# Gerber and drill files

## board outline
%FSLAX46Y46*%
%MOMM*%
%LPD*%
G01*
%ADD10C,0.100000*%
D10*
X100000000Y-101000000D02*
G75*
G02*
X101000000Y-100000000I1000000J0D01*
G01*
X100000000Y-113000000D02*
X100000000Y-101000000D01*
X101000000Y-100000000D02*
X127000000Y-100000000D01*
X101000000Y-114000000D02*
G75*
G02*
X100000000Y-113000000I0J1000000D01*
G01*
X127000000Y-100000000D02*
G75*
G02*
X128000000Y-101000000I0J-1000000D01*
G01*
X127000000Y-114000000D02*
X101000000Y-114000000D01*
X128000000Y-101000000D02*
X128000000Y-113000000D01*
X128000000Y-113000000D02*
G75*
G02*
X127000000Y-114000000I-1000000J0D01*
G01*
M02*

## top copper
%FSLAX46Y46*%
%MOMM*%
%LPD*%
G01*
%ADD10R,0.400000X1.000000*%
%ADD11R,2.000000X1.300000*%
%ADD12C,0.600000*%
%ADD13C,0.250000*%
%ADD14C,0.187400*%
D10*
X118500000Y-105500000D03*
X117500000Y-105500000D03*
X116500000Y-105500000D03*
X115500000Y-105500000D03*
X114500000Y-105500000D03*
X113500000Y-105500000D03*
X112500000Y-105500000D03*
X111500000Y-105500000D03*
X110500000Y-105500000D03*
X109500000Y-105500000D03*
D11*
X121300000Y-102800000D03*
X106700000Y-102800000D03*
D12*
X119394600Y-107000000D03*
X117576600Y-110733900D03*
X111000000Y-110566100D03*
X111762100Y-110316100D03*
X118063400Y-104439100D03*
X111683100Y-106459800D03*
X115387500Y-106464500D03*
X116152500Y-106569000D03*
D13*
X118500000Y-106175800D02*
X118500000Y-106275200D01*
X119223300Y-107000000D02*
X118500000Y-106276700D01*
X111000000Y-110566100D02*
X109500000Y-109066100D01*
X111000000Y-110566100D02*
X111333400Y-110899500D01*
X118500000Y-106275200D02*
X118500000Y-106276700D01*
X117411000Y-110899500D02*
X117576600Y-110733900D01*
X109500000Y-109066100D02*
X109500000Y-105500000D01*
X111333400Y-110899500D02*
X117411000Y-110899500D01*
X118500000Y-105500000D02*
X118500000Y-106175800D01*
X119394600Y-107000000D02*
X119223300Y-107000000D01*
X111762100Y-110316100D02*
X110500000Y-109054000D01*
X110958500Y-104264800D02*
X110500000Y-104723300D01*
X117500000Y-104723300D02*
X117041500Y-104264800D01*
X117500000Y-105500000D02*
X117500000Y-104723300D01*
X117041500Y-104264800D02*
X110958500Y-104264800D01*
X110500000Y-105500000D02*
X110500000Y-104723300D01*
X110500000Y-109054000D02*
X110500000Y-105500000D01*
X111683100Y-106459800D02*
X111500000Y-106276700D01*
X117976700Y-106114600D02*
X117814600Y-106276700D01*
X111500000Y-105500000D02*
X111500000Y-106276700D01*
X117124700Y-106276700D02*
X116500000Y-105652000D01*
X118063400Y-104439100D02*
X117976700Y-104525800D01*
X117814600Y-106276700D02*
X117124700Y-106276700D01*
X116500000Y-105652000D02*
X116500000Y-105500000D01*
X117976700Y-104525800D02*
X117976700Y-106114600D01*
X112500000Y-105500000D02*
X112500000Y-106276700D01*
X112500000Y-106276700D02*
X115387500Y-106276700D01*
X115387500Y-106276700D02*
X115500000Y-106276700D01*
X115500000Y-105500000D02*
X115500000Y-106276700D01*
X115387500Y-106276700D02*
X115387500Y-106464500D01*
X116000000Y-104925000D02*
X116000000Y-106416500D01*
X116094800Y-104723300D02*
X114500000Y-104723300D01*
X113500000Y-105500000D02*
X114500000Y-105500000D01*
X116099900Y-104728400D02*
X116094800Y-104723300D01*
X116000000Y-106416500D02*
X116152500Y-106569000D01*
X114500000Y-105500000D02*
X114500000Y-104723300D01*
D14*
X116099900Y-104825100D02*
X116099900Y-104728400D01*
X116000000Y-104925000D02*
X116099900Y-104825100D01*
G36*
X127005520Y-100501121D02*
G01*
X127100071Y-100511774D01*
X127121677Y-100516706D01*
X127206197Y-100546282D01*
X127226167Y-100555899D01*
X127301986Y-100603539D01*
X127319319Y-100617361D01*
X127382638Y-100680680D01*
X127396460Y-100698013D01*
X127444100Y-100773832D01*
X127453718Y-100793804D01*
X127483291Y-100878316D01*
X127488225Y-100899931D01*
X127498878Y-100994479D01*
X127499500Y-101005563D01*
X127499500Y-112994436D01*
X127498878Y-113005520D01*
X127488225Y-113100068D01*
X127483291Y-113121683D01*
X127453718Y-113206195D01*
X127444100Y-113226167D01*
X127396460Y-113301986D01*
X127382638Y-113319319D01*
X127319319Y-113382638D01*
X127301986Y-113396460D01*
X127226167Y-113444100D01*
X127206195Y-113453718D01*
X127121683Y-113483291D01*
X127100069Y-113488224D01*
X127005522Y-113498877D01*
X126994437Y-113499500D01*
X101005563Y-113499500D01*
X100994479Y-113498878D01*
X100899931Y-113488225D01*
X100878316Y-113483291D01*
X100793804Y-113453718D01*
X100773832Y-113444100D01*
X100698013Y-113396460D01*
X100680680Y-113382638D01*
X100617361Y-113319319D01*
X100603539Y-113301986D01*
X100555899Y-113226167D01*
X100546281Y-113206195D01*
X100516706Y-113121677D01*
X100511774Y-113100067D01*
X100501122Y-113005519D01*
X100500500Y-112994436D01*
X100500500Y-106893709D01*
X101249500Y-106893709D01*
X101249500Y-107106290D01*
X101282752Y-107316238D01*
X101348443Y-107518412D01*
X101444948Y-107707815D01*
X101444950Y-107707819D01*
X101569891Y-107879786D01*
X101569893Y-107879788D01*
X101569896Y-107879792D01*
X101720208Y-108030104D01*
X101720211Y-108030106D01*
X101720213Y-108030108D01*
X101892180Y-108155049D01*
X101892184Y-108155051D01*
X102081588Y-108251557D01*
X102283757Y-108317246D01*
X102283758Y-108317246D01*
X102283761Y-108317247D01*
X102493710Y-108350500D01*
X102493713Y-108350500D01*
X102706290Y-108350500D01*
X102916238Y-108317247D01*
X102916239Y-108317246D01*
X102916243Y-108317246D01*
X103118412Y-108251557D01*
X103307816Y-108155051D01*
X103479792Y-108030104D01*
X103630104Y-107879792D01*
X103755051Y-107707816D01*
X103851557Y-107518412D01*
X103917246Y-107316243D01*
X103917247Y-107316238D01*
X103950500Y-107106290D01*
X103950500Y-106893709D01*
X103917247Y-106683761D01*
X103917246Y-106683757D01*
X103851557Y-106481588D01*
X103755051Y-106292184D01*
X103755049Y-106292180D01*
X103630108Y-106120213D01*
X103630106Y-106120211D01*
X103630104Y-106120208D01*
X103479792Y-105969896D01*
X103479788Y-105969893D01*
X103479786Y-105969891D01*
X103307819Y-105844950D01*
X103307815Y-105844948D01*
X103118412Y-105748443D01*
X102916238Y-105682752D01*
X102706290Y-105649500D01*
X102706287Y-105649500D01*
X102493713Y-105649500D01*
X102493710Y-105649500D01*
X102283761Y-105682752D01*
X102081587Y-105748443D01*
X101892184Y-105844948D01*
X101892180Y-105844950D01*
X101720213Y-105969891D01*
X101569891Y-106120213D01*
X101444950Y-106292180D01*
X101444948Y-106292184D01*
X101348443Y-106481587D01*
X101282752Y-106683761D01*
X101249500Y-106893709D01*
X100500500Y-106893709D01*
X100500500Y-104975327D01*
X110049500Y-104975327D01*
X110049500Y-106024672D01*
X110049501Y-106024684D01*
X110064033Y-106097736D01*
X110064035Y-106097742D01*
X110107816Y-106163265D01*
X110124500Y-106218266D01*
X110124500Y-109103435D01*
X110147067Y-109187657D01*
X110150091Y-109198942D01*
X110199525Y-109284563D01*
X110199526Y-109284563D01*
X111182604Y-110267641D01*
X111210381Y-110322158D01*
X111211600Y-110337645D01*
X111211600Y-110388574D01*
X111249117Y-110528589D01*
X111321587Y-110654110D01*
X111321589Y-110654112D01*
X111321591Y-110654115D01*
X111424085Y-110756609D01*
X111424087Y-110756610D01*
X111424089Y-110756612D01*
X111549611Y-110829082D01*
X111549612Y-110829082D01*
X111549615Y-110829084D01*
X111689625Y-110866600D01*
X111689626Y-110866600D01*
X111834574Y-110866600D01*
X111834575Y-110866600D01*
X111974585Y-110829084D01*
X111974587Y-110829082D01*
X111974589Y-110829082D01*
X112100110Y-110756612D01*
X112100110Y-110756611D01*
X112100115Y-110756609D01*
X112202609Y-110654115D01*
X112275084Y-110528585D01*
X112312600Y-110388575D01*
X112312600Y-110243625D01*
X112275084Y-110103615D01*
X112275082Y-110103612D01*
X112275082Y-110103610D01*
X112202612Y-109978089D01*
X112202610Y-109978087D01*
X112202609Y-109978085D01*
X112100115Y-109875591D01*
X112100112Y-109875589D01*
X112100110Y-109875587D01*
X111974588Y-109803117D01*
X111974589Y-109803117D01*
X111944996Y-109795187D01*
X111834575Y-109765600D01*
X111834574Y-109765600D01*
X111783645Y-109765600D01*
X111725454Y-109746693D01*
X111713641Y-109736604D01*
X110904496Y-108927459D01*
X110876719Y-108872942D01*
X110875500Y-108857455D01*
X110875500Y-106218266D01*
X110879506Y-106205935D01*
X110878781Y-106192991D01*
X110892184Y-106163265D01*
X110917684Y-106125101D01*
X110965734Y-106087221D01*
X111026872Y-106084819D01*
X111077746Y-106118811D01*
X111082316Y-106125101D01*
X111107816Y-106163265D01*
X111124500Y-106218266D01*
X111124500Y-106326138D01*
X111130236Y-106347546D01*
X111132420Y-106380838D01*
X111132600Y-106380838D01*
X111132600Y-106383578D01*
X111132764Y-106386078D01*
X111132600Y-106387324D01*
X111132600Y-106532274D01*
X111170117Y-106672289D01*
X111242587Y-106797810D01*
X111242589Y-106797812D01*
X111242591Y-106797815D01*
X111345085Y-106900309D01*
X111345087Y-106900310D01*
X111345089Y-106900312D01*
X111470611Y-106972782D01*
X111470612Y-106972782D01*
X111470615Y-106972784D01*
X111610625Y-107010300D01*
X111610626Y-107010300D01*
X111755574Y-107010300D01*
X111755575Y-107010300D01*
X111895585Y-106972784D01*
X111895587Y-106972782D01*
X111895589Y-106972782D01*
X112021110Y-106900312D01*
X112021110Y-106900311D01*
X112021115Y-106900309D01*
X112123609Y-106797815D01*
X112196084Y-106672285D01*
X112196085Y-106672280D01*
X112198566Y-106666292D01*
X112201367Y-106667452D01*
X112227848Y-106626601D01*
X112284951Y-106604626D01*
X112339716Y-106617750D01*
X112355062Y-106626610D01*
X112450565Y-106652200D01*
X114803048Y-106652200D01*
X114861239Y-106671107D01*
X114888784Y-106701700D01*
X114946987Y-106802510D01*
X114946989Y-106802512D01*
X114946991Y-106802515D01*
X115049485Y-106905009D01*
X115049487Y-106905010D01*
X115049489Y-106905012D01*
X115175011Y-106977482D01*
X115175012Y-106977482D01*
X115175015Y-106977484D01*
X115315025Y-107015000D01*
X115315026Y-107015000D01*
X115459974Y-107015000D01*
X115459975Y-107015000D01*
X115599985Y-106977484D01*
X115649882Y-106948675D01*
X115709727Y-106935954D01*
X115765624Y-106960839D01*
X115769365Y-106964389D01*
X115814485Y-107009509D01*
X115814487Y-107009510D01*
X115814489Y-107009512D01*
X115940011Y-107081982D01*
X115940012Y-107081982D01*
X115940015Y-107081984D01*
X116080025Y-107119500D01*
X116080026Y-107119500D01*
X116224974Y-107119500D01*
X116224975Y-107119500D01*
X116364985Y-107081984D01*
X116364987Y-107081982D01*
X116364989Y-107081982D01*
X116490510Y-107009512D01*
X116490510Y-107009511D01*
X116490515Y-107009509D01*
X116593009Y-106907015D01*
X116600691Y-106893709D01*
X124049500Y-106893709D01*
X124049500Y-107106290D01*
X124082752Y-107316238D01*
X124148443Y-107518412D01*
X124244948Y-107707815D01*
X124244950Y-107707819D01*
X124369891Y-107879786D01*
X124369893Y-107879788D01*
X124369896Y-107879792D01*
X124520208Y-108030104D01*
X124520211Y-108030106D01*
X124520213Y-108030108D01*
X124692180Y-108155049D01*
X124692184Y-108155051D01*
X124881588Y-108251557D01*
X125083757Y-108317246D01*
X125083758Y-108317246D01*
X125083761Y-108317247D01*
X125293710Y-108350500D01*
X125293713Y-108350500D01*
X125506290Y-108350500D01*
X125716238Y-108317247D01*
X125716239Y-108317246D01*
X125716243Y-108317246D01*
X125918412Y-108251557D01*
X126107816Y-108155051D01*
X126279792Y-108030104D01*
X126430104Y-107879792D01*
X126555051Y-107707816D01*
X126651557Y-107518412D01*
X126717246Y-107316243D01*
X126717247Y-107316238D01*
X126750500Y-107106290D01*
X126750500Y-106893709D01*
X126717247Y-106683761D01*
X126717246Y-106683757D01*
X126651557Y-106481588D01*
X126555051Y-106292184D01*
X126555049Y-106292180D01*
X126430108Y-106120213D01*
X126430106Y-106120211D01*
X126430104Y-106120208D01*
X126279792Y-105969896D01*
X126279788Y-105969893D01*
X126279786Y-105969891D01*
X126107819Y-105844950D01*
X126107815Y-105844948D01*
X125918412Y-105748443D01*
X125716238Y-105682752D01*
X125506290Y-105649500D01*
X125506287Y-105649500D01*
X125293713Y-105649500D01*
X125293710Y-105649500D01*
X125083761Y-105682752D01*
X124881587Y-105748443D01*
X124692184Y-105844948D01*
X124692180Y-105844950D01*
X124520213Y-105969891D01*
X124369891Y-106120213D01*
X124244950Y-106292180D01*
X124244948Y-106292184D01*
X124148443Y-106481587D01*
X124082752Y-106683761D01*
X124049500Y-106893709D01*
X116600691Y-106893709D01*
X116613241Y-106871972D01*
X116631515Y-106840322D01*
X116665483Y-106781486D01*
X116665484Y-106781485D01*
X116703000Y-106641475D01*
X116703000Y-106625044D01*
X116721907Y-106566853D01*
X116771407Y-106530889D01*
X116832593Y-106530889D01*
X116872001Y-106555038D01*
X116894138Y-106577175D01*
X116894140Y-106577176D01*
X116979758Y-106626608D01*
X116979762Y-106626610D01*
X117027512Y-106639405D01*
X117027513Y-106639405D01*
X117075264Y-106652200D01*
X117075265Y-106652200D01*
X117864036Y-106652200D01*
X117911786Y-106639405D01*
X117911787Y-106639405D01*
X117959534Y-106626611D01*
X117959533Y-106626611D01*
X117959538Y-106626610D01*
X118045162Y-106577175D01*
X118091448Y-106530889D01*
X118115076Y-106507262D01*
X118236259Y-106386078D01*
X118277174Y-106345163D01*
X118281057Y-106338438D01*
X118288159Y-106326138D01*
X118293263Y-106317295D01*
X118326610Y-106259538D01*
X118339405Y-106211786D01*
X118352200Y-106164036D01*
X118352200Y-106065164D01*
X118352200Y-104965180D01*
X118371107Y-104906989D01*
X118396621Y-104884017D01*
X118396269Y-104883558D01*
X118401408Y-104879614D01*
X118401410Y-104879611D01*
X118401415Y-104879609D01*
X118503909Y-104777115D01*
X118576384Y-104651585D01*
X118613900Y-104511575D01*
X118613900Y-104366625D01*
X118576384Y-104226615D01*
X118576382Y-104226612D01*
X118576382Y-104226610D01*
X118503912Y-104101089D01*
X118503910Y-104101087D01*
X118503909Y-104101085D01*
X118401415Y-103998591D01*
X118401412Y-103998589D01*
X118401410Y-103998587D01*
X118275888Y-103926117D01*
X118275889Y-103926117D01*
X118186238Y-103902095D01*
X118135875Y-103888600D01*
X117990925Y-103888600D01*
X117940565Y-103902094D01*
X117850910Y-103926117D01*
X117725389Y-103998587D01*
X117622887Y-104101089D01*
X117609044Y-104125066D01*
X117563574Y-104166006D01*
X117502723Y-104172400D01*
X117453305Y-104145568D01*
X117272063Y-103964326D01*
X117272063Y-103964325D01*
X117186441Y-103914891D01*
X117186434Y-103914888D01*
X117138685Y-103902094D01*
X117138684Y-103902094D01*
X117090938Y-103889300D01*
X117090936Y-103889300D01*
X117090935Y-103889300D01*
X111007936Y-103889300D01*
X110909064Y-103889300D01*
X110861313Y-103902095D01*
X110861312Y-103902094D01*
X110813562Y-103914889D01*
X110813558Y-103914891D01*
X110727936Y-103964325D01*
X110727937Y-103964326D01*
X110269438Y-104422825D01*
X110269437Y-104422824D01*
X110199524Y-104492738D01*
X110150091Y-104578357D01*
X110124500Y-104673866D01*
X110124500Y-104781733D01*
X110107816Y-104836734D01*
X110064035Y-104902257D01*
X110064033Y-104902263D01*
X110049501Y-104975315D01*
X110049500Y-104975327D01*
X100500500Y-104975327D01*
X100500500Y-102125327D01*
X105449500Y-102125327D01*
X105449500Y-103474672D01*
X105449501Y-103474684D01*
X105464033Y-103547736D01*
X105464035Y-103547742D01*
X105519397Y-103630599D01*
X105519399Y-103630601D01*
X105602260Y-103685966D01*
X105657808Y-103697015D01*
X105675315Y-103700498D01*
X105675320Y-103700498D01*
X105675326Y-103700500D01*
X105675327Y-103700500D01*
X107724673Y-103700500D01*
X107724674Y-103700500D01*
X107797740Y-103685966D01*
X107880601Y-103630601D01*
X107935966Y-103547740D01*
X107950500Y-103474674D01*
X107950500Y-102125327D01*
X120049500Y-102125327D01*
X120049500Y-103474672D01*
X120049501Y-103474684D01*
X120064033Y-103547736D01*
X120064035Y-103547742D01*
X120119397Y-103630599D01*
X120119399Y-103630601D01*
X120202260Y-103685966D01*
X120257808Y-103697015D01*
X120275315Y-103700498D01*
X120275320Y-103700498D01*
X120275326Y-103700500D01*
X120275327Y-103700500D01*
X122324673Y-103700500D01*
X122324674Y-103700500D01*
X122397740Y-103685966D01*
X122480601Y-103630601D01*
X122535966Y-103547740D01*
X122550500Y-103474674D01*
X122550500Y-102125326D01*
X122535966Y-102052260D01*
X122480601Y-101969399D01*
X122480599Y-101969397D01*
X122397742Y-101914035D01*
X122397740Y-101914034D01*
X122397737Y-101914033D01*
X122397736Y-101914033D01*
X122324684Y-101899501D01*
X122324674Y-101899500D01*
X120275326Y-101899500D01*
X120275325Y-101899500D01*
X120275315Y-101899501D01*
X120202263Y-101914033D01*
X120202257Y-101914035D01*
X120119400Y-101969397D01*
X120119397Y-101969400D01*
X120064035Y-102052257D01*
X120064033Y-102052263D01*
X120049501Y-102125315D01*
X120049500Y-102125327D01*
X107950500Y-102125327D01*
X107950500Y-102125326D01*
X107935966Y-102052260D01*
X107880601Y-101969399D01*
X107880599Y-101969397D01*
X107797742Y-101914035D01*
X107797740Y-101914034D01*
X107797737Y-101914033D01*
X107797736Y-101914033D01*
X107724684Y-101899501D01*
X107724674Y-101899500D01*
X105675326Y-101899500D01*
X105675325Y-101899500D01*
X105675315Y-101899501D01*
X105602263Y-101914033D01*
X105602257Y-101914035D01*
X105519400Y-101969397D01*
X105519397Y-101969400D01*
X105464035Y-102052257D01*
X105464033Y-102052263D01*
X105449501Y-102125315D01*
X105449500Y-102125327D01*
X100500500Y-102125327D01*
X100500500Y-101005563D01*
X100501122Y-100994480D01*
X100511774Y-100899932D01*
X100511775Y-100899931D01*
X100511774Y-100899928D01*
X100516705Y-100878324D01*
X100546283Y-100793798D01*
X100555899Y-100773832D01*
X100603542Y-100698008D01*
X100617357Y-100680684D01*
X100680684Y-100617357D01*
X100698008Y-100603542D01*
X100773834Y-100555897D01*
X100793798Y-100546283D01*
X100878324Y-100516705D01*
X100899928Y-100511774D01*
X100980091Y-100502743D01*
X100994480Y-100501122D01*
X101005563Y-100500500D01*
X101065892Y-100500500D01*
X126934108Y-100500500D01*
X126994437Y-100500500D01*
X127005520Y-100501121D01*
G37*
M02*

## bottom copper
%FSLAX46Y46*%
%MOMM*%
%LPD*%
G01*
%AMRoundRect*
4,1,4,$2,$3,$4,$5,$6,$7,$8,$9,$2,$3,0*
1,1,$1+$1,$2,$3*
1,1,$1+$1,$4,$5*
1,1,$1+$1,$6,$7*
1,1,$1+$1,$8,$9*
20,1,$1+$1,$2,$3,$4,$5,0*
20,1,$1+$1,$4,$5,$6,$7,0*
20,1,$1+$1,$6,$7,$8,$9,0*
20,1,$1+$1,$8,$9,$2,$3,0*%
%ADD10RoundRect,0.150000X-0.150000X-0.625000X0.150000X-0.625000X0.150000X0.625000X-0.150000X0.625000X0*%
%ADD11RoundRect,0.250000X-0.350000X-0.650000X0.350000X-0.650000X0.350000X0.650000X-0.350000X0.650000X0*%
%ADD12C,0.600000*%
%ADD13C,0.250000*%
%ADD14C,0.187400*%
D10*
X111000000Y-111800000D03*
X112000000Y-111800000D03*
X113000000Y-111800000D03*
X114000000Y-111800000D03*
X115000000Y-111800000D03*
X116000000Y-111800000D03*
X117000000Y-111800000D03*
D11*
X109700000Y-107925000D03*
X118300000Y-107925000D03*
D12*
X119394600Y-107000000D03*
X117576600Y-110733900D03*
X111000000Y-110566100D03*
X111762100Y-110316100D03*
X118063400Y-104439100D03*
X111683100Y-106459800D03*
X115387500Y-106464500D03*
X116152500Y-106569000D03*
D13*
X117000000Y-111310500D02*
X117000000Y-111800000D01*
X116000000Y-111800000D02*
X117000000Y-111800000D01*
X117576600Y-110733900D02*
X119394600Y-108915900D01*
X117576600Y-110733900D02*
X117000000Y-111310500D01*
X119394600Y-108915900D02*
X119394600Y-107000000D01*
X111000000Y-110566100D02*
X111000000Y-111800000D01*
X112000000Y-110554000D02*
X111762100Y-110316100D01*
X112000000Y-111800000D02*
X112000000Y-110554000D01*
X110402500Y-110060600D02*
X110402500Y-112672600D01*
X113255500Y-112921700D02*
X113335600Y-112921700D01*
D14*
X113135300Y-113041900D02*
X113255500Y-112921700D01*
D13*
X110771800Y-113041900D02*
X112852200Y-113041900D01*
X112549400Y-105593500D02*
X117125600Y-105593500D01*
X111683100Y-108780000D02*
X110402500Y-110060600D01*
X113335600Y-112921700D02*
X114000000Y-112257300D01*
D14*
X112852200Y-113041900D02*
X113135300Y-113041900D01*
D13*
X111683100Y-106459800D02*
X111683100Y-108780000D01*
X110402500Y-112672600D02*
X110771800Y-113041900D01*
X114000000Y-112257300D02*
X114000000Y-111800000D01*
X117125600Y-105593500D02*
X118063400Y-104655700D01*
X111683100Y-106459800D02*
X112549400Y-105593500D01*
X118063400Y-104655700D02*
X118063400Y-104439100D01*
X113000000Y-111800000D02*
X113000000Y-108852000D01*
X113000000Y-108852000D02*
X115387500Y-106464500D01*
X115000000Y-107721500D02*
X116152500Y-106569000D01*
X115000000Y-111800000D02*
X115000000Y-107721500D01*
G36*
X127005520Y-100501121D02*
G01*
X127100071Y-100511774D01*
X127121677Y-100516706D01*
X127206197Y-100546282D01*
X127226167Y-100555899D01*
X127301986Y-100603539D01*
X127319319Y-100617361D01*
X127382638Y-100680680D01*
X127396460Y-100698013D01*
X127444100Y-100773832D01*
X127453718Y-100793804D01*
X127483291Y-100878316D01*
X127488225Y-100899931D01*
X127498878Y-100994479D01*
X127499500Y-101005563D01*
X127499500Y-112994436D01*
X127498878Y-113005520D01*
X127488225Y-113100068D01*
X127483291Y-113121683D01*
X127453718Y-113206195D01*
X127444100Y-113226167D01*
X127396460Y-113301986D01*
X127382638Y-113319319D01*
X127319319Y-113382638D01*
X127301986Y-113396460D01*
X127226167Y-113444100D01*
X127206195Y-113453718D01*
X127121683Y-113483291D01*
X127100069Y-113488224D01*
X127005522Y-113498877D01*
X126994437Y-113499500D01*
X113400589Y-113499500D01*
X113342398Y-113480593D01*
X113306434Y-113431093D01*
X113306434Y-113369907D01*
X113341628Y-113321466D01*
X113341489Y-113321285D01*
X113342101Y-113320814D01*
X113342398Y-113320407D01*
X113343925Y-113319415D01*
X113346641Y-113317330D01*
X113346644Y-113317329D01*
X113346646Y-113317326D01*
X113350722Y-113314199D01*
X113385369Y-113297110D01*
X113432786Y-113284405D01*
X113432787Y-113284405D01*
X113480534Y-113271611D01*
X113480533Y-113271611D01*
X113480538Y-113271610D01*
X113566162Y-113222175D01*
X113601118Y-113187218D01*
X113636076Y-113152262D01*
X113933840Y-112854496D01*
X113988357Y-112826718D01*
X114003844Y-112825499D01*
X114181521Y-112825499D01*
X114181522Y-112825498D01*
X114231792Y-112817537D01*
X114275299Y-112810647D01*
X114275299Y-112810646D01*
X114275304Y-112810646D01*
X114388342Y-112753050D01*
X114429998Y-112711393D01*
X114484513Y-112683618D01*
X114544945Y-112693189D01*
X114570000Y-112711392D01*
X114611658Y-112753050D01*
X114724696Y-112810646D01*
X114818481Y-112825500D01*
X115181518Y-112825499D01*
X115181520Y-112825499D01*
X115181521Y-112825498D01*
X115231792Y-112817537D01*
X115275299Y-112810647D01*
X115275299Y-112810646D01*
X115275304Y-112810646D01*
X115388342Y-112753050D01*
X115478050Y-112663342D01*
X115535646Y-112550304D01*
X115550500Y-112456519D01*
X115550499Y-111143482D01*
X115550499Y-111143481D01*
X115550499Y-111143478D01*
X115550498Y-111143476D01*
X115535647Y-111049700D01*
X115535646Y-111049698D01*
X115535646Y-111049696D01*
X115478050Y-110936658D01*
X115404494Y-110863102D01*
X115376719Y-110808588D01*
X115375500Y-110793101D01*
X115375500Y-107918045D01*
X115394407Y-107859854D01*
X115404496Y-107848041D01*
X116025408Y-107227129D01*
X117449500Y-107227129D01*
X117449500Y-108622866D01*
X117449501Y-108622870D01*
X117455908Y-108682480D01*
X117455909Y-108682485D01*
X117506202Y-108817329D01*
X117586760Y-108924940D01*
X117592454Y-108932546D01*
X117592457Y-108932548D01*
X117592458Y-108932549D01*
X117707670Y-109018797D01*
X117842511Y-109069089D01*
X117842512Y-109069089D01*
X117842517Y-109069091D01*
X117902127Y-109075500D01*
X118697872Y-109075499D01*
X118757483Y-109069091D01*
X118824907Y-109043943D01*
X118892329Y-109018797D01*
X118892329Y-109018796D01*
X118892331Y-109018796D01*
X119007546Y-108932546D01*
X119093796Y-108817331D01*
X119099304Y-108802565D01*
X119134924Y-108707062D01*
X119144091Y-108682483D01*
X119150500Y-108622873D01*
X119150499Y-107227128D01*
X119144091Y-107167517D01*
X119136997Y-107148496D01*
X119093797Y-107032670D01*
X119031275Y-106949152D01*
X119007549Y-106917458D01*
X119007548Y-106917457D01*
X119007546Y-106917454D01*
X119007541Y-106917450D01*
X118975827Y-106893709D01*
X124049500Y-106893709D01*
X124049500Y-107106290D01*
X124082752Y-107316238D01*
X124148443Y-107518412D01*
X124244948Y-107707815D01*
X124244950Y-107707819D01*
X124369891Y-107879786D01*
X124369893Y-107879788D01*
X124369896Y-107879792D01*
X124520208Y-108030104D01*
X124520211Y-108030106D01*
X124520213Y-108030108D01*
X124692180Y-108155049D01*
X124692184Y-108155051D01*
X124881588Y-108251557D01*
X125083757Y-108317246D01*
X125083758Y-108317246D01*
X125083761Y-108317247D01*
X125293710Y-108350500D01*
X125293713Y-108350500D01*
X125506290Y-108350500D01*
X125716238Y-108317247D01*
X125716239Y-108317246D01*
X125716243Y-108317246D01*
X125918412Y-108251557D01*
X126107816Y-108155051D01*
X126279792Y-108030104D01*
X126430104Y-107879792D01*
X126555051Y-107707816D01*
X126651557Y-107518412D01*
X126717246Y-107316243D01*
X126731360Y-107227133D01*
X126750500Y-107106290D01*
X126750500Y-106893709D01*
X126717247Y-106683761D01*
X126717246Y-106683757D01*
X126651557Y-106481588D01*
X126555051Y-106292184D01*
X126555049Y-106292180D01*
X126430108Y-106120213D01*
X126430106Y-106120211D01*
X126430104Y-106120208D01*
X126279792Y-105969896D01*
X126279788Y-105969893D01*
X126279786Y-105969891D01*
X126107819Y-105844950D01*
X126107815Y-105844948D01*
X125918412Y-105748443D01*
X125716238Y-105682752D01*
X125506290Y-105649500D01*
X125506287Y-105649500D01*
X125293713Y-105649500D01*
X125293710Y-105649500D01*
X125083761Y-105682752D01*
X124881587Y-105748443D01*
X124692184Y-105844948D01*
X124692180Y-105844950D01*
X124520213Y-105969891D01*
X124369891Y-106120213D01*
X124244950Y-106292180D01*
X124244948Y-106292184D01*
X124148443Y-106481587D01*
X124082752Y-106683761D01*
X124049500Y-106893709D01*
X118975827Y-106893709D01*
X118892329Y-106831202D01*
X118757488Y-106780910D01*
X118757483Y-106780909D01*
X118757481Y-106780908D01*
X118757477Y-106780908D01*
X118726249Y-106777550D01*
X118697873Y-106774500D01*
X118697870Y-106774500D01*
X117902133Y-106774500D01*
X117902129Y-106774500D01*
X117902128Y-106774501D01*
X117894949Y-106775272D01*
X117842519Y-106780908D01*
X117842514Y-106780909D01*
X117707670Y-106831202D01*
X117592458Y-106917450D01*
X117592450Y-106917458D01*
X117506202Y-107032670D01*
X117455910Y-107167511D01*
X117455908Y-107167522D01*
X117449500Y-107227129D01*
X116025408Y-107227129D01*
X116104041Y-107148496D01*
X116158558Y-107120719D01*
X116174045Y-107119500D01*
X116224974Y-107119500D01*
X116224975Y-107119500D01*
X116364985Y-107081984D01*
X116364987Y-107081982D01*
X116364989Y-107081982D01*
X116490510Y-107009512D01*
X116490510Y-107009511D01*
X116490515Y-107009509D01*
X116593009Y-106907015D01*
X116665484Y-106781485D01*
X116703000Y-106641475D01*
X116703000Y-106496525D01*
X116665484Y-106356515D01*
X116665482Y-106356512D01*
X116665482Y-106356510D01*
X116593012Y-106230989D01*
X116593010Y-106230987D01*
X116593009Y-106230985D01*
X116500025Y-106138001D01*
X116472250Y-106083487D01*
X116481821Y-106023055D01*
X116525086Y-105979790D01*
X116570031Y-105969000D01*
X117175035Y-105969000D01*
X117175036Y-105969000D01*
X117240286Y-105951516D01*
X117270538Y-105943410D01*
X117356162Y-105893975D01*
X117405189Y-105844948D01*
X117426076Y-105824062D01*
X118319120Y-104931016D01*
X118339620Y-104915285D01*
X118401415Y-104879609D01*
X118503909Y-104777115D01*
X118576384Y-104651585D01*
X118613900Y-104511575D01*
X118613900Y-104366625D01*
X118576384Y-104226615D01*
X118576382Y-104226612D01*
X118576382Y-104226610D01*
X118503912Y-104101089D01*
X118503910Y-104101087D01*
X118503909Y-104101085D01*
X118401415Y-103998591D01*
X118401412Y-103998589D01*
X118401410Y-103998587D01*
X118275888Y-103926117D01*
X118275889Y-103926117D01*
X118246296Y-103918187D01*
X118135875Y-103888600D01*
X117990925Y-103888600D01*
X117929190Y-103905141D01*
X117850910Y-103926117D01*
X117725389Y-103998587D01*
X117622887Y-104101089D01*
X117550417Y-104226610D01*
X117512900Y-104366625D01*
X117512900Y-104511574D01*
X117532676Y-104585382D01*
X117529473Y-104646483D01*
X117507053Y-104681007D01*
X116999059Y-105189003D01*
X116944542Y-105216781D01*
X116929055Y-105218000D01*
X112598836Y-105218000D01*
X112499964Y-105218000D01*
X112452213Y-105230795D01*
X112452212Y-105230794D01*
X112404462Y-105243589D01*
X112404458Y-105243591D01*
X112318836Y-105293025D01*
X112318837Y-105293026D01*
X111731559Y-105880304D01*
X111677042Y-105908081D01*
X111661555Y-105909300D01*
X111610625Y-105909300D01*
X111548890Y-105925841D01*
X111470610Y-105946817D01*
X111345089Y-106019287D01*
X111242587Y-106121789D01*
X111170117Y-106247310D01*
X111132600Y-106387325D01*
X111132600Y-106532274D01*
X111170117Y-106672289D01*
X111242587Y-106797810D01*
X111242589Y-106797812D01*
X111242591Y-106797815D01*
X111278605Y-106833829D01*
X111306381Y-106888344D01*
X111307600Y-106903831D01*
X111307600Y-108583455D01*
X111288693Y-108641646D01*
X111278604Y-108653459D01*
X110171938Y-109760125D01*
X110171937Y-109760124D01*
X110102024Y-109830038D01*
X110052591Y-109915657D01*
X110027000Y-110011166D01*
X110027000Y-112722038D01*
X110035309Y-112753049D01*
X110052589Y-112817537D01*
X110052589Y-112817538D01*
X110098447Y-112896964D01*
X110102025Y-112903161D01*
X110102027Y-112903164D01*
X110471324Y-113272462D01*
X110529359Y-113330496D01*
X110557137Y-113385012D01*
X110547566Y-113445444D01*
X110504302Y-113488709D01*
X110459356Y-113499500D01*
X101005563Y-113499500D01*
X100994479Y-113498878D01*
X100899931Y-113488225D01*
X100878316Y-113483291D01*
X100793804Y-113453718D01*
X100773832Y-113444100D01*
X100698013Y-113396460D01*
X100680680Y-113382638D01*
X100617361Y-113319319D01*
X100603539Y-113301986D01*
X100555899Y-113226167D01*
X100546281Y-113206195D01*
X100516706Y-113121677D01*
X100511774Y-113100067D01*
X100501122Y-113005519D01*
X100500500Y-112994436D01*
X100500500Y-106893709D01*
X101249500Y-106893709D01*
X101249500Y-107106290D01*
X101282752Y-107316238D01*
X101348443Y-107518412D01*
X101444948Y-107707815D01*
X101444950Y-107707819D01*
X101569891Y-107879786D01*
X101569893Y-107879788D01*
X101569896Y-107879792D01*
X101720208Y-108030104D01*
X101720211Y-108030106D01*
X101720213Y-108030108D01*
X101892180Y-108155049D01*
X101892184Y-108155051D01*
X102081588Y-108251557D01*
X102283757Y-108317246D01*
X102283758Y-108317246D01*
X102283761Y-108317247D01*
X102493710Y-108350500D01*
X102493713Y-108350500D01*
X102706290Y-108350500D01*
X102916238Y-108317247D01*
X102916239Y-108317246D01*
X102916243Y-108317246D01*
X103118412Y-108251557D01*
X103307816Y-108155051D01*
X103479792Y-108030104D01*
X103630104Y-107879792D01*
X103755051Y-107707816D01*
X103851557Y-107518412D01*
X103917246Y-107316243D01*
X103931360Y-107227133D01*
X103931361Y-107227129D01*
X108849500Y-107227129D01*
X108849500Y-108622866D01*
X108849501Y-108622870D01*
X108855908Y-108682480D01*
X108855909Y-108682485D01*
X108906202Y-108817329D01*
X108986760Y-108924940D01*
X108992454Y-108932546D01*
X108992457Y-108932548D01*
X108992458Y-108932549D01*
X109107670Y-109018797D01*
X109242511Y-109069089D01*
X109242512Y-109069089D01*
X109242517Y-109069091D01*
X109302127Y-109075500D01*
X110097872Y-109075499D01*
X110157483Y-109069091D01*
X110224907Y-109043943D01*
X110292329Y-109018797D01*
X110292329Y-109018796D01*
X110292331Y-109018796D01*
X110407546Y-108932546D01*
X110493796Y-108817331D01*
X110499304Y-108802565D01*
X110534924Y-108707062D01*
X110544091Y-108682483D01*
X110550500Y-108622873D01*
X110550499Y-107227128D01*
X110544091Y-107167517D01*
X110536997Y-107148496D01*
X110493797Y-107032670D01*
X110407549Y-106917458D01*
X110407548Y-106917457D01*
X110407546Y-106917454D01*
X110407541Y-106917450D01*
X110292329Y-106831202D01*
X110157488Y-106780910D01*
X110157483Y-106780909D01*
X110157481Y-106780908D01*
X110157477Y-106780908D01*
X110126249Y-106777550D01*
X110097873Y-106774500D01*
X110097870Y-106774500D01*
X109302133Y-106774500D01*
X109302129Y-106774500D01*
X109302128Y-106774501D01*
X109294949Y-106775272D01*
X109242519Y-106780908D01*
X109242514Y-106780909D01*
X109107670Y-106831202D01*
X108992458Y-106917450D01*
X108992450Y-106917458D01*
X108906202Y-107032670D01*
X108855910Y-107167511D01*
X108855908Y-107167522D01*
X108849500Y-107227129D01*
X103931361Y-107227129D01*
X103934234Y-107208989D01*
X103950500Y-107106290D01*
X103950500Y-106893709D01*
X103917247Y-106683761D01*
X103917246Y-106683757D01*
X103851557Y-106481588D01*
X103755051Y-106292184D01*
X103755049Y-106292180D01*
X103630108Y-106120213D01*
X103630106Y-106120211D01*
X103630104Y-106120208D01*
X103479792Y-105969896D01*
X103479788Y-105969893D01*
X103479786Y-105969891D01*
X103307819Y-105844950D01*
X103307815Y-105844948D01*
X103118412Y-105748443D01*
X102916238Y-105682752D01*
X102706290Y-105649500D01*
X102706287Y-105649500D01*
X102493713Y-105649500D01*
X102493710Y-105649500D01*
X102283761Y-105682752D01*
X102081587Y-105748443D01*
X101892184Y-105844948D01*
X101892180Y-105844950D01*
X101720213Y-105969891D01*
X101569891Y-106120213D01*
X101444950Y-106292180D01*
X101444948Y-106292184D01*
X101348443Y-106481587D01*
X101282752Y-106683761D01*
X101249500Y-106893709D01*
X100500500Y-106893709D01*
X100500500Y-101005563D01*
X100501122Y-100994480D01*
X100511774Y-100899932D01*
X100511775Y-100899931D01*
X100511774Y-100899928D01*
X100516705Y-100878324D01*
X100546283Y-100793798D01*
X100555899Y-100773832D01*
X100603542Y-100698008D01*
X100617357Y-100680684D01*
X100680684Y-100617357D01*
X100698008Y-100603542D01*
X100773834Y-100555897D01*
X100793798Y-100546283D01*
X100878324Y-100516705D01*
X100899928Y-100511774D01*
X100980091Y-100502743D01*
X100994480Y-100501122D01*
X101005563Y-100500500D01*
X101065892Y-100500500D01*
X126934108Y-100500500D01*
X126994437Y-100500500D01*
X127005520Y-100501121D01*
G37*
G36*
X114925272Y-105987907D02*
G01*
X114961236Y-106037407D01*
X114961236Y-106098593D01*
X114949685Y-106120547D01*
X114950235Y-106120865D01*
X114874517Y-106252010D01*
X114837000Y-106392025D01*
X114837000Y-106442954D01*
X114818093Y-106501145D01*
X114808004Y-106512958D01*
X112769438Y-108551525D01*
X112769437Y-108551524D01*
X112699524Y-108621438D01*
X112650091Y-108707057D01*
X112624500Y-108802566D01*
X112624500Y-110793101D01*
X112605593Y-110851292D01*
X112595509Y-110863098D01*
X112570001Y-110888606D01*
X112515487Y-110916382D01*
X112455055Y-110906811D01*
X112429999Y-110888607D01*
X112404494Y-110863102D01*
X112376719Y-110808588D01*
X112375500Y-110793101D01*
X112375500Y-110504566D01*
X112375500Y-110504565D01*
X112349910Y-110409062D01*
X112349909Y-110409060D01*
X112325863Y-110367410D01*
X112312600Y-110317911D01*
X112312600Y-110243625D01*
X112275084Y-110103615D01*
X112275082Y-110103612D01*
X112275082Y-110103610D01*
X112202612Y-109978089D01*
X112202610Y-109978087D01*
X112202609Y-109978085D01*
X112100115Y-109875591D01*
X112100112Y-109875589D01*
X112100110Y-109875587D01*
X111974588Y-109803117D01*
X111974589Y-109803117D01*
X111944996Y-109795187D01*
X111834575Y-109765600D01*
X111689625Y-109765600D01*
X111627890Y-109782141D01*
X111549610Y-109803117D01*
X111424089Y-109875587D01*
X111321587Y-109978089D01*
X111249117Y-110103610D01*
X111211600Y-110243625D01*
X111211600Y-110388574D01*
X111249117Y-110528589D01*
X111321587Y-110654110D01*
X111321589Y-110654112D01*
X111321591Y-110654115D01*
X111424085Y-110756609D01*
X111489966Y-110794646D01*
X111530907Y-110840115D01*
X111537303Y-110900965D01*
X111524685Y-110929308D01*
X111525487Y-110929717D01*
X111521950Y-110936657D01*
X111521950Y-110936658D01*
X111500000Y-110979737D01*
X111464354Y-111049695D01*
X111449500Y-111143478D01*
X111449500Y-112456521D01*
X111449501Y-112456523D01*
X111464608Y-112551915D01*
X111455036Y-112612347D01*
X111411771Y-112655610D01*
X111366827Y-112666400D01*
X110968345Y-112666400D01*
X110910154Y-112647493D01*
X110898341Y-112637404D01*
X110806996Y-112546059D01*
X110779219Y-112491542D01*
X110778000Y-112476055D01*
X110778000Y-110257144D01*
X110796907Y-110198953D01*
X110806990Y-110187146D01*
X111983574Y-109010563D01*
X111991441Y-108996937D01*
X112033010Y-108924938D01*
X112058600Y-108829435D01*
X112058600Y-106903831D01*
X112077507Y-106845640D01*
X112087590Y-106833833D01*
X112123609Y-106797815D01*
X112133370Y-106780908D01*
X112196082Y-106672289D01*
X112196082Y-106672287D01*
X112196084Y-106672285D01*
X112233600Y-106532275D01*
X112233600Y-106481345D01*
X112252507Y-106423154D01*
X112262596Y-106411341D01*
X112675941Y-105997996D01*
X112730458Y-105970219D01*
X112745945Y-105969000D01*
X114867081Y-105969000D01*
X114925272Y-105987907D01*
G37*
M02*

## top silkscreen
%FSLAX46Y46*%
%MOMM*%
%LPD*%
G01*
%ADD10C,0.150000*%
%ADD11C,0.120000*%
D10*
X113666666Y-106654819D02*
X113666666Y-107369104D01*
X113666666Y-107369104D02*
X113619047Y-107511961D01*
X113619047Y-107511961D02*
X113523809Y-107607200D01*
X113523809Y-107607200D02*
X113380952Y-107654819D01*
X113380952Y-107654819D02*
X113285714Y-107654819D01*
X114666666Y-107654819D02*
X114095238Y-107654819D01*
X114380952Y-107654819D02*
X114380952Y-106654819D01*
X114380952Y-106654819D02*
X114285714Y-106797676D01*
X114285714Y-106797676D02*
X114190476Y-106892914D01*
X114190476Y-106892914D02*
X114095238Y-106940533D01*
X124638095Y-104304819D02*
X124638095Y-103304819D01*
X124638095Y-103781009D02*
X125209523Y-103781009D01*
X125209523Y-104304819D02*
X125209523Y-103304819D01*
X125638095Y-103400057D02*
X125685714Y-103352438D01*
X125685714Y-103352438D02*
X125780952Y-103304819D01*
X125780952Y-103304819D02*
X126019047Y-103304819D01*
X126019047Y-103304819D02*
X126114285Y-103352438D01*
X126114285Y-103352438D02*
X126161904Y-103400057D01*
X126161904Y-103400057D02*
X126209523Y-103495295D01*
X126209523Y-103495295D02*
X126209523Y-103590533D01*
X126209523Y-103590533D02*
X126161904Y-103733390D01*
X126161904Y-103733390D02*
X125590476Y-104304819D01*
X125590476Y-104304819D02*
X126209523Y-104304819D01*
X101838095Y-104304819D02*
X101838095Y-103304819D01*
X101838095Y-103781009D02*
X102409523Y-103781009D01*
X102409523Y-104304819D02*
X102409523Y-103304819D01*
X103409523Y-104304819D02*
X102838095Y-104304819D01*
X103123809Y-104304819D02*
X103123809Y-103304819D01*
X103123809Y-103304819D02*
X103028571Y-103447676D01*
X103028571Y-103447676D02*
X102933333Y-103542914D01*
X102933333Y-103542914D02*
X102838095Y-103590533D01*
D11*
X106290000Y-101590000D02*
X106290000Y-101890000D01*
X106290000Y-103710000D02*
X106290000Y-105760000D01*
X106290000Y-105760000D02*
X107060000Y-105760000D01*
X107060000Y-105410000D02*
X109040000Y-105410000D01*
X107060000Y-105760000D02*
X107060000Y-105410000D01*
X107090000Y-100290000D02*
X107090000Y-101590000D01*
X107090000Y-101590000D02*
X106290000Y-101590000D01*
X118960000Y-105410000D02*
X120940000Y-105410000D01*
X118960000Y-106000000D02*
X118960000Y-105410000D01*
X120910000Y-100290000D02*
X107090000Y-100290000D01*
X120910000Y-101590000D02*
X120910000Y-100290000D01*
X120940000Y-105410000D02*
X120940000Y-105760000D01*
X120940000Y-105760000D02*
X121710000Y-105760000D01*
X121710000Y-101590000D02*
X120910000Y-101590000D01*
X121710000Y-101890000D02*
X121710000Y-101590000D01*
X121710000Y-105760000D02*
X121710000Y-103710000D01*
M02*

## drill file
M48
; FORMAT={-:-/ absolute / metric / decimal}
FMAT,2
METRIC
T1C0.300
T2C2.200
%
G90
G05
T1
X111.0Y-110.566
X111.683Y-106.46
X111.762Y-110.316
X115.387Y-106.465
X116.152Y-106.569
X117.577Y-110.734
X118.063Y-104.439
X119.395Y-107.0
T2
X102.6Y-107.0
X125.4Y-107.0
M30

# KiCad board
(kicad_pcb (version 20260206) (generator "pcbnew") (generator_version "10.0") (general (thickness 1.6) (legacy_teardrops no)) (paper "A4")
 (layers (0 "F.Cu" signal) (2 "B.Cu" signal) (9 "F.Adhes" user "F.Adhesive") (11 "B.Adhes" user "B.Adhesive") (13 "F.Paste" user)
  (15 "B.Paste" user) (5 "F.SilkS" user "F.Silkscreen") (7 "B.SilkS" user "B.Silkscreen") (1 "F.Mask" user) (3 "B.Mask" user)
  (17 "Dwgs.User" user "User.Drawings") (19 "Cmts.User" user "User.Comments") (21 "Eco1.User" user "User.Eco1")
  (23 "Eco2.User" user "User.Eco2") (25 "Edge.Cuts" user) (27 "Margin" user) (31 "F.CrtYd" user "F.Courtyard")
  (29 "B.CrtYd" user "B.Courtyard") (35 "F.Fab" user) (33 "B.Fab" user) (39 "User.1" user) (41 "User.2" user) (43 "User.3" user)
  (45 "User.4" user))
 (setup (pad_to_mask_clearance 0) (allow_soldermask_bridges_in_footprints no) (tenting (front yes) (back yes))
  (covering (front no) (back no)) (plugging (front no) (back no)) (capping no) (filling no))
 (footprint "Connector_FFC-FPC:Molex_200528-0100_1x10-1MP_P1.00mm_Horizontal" (layer "F.Cu") (at 114 104.59 180)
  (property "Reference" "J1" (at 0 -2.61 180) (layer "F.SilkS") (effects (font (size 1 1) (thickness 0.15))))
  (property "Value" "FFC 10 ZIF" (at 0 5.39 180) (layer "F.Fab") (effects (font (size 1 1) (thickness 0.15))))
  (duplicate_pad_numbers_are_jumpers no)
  (fp_line (start 7.71 3) (end 7.71 2.7) (stroke (width 0.12) (type solid)) (layer "F.SilkS"))
  (fp_line (start 7.71 0.88) (end 7.71 -1.17) (stroke (width 0.12) (type solid)) (layer "F.SilkS"))
  (fp_line (start 7.71 -1.17) (end 6.94 -1.17) (stroke (width 0.12) (type solid)) (layer "F.SilkS"))
  (fp_line (start 6.94 -0.82) (end 4.96 -0.82) (stroke (width 0.12) (type solid)) (layer "F.SilkS"))
  (fp_line (start 6.94 -1.17) (end 6.94 -0.82) (stroke (width 0.12) (type solid)) (layer "F.SilkS"))
  (fp_line (start 6.91 4.3) (end 6.91 3) (stroke (width 0.12) (type solid)) (layer "F.SilkS"))
  (fp_line (start 6.91 3) (end 7.71 3) (stroke (width 0.12) (type solid)) (layer "F.SilkS"))
  (fp_line (start -4.96 -0.82) (end -6.94 -0.82) (stroke (width 0.12) (type solid)) (layer "F.SilkS"))
  (fp_line (start -4.96 -1.41) (end -4.96 -0.82) (stroke (width 0.12) (type solid)) (layer "F.SilkS"))
  (fp_line (start -6.91 4.3) (end 6.91 4.3) (stroke (width 0.12) (type solid)) (layer "F.SilkS"))
  (fp_line (start -6.91 3) (end -6.91 4.3) (stroke (width 0.12) (type solid)) (layer "F.SilkS"))
  (fp_line (start -6.94 -0.82) (end -6.94 -1.17) (stroke (width 0.12) (type solid)) (layer "F.SilkS"))
  (fp_line (start -6.94 -1.17) (end -7.71 -1.17) (stroke (width 0.12) (type solid)) (layer "F.SilkS"))
  (fp_line (start -7.71 3) (end -6.91 3) (stroke (width 0.12) (type solid)) (layer "F.SilkS"))
  (fp_line (start -7.71 2.7) (end -7.71 3) (stroke (width 0.12) (type solid)) (layer "F.SilkS"))
  (fp_line (start -7.71 -1.17) (end -7.71 0.88) (stroke (width 0.12) (type solid)) (layer "F.SilkS"))
  (pad "1" smd rect (at -4.5 -0.91 180) (size 0.4 1) (layers "F.Cu" "F.Mask" "F.Paste") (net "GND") (zone_connect 2))
  (pad "2" smd rect (at -3.5 -0.91 180) (size 0.4 1) (layers "F.Cu" "F.Mask" "F.Paste") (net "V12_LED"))
  (pad "3" smd rect (at -2.5 -0.91 180) (size 0.4 1) (layers "F.Cu" "F.Mask" "F.Paste") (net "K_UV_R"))
  (pad "4" smd rect (at -1.5 -0.91 180) (size 0.4 1) (layers "F.Cu" "F.Mask" "F.Paste") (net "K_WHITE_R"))
  (pad "5" smd rect (at -0.5 -0.91 180) (size 0.4 1) (layers "F.Cu" "F.Mask" "F.Paste") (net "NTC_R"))
  (pad "6" smd rect (at 0.5 -0.91 180) (size 0.4 1) (layers "F.Cu" "F.Mask" "F.Paste") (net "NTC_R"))
  (pad "7" smd rect (at 1.5 -0.91 180) (size 0.4 1) (layers "F.Cu" "F.Mask" "F.Paste") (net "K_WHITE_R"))
  (pad "8" smd rect (at 2.5 -0.91 180) (size 0.4 1) (layers "F.Cu" "F.Mask" "F.Paste") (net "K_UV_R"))
  (pad "9" smd rect (at 3.5 -0.91 180) (size 0.4 1) (layers "F.Cu" "F.Mask" "F.Paste") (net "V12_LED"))
  (pad "10" smd rect (at 4.5 -0.91 180) (size 0.4 1) (layers "F.Cu" "F.Mask" "F.Paste") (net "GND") (zone_connect 2))
  (pad "MP" smd rect (at -7.3 1.79 180) (size 2 1.3) (layers "F.Cu" "F.Mask" "F.Paste") (zone_connect 2))
  (pad "MP" smd rect (at 7.3 1.79 180) (size 2 1.3) (layers "F.Cu" "F.Mask" "F.Paste") (zone_connect 2)))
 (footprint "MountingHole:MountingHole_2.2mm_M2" (layer "F.Cu") (at 125.4 107)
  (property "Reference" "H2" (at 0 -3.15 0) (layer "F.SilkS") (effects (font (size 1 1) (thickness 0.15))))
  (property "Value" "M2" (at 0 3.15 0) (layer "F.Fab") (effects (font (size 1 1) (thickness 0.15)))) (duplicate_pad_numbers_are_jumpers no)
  (pad "" np_thru_hole circle (at 0 0) (size 2.2 2.2) (drill 2.2) (layers "*.Cu" "*.Mask") (zone_connect 2)))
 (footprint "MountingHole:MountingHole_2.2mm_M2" (layer "F.Cu") (at 102.6 107)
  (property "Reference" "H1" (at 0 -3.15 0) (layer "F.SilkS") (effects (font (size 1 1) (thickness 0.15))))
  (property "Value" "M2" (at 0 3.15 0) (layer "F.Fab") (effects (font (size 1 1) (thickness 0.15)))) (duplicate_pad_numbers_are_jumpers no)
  (pad "" np_thru_hole circle (at 0 0) (size 2.2 2.2) (drill 2.2) (layers "*.Cu" "*.Mask") (zone_connect 2)))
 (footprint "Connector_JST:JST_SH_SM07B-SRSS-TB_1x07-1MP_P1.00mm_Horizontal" (layer "B.Cu") (at 114 109.8)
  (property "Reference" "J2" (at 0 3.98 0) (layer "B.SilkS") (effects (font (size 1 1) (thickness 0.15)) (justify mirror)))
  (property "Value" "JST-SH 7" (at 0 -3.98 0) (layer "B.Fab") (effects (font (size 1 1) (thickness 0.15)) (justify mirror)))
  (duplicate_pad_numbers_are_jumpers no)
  (pad "1" smd roundrect (at -3 2) (size 0.6 1.55) (layers "B.Cu" "B.Mask" "B.Paste") (roundrect_rratio 0.25) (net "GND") (zone_connect 2))
  (pad "2" smd roundrect (at -2 2) (size 0.6 1.55) (layers "B.Cu" "B.Mask" "B.Paste") (roundrect_rratio 0.25) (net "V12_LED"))
  (pad "3" smd roundrect (at -1 2) (size 0.6 1.55) (layers "B.Cu" "B.Mask" "B.Paste") (roundrect_rratio 0.25) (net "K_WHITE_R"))
  (pad "4" smd roundrect (at 0 2) (size 0.6 1.55) (layers "B.Cu" "B.Mask" "B.Paste") (roundrect_rratio 0.25) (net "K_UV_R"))
  (pad "5" smd roundrect (at 1 2) (size 0.6 1.55) (layers "B.Cu" "B.Mask" "B.Paste") (roundrect_rratio 0.25) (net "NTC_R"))
  (pad "6" smd roundrect (at 2 2) (size 0.6 1.55) (layers "B.Cu" "B.Mask" "B.Paste") (roundrect_rratio 0.25) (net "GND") (zone_connect 2))
  (pad "7" smd roundrect (at 3 2) (size 0.6 1.55) (layers "B.Cu" "B.Mask" "B.Paste") (roundrect_rratio 0.25) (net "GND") (zone_connect 2))
  (pad "MP" smd roundrect (at -4.3 -1.875) (size 1.2 1.8) (layers "B.Cu" "B.Mask" "B.Paste") (roundrect_rratio 0.208333) (zone_connect 2))
  (pad "MP" smd roundrect (at 4.3 -1.875) (size 1.2 1.8) (layers "B.Cu" "B.Mask" "B.Paste") (roundrect_rratio 0.208333) (zone_connect 2)))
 (gr_arc (start 100 101) (mid 100.292893 100.292893) (end 101 100) (stroke (width 0.1) (type default)) (layer "Edge.Cuts"))
 (gr_line (start 100 113) (end 100 101) (stroke (width 0.1) (type default)) (layer "Edge.Cuts"))
 (gr_line (start 101 100) (end 127 100) (stroke (width 0.1) (type default)) (layer "Edge.Cuts"))
 (gr_arc (start 101 114) (mid 100.292893 113.707107) (end 100 113) (stroke (width 0.1) (type default)) (layer "Edge.Cuts"))
 (gr_arc (start 127 100) (mid 127.707107 100.292893) (end 128 101) (stroke (width 0.1) (type default)) (layer "Edge.Cuts"))
 (gr_line (start 127 114) (end 101 114) (stroke (width 0.1) (type default)) (layer "Edge.Cuts"))
 (gr_line (start 128 101) (end 128 113) (stroke (width 0.1) (type default)) (layer "Edge.Cuts"))
 (gr_arc (start 128 113) (mid 127.707107 113.707107) (end 127 114) (stroke (width 0.1) (type default)) (layer "Edge.Cuts"))
 (segment (start 118.5 106.1758) (end 118.5 106.2752) (width 0.25) (layer "F.Cu") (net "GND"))
 (segment (start 119.2233 107) (end 118.5 106.2767) (width 0.25) (layer "F.Cu") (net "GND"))
 (segment (start 111 110.5661) (end 109.5 109.0661) (width 0.25) (layer "F.Cu") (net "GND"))
 (segment (start 111 110.5661) (end 111.3334 110.8995) (width 0.25) (layer "F.Cu") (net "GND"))
 (segment (start 118.5 106.2752) (end 118.5 106.2767) (width 0.25) (layer "F.Cu") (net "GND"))
 (segment (start 117.411 110.8995) (end 117.5766 110.7339) (width 0.25) (layer "F.Cu") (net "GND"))
 (segment (start 109.5 109.0661) (end 109.5 105.5) (width 0.25) (layer "F.Cu") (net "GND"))
 (segment (start 111.3334 110.8995) (end 117.411 110.8995) (width 0.25) (layer "F.Cu") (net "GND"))
 (segment (start 118.5 105.5) (end 118.5 106.1758) (width 0.25) (layer "F.Cu") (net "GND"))
 (segment (start 119.3946 107) (end 119.2233 107) (width 0.25) (layer "F.Cu") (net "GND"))
 (via (at 119.3946 107) (size 0.6) (drill 0.3) (layers "F.Cu" "B.Cu") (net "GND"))
 (via (at 117.5766 110.7339) (size 0.6) (drill 0.3) (layers "F.Cu" "B.Cu") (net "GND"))
 (via (at 111 110.5661) (size 0.6) (drill 0.3) (layers "F.Cu" "B.Cu") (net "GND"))
 (segment (start 117 111.3105) (end 117 111.8) (width 0.25) (layer "B.Cu") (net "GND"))
 (segment (start 116 111.8) (end 117 111.8) (width 0.25) (layer "B.Cu") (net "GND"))
 (segment (start 117.5766 110.7339) (end 119.3946 108.9159) (width 0.25) (layer "B.Cu") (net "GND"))
 (segment (start 117.5766 110.7339) (end 117 111.3105) (width 0.25) (layer "B.Cu") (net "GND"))
 (segment (start 119.3946 108.9159) (end 119.3946 107) (width 0.25) (layer "B.Cu") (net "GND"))
 (segment (start 111 110.5661) (end 111 111.8) (width 0.25) (layer "B.Cu") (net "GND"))
 (segment (start 111.7621 110.3161) (end 110.5 109.054) (width 0.25) (layer "F.Cu") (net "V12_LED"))
 (segment (start 110.9585 104.2648) (end 110.5 104.7233) (width 0.25) (layer "F.Cu") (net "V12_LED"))
 (segment (start 117.5 104.7233) (end 117.0415 104.2648) (width 0.25) (layer "F.Cu") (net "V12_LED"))
 (segment (start 117.5 105.5) (end 117.5 104.7233) (width 0.25) (layer "F.Cu") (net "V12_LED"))
 (segment (start 117.0415 104.2648) (end 110.9585 104.2648) (width 0.25) (layer "F.Cu") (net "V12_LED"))
 (segment (start 110.5 105.5) (end 110.5 104.7233) (width 0.25) (layer "F.Cu") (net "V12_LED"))
 (segment (start 110.5 109.054) (end 110.5 105.5) (width 0.25) (layer "F.Cu") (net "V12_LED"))
 (via (at 111.7621 110.3161) (size 0.6) (drill 0.3) (layers "F.Cu" "B.Cu") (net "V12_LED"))
 (segment (start 112 110.554) (end 111.7621 110.3161) (width 0.25) (layer "B.Cu") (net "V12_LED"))
 (segment (start 112 111.8) (end 112 110.554) (width 0.25) (layer "B.Cu") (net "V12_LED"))
 (segment (start 111.6831 106.4598) (end 111.5 106.2767) (width 0.25) (layer "F.Cu") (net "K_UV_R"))
 (segment (start 117.9767 106.1146) (end 117.8146 106.2767) (width 0.25) (layer "F.Cu") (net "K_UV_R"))
 (segment (start 111.5 105.5) (end 111.5 106.2767) (width 0.25) (layer "F.Cu") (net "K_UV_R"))
 (segment (start 117.1247 106.2767) (end 116.5 105.652) (width 0.25) (layer "F.Cu") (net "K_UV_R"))
 (segment (start 118.0634 104.4391) (end 117.9767 104.5258) (width 0.25) (layer "F.Cu") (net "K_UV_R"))
 (segment (start 117.8146 106.2767) (end 117.1247 106.2767) (width 0.25) (layer "F.Cu") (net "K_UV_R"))
 (segment (start 116.5 105.652) (end 116.5 105.5) (width 0.25) (layer "F.Cu") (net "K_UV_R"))
 (segment (start 117.9767 104.5258) (end 117.9767 106.1146) (width 0.25) (layer "F.Cu") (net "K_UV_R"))
 (via (at 118.0634 104.4391) (size 0.6) (drill 0.3) (layers "F.Cu" "B.Cu") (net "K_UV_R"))
 (via (at 111.6831 106.4598) (size 0.6) (drill 0.3) (layers "F.Cu" "B.Cu") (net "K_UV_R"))
 (segment (start 110.4025 110.0606) (end 110.4025 112.6726) (width 0.25) (layer "B.Cu") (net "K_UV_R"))
 (segment (start 113.2555 112.9217) (end 113.3356 112.9217) (width 0.25) (layer "B.Cu") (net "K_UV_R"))
 (segment (start 113.1353 113.0419) (end 113.2555 112.9217) (width 0.1874) (layer "B.Cu") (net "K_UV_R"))
 (segment (start 110.7718 113.0419) (end 112.8522 113.0419) (width 0.25) (layer "B.Cu") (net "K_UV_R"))
 (segment (start 112.5494 105.5935) (end 117.1256 105.5935) (width 0.25) (layer "B.Cu") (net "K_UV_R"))
 (segment (start 111.6831 108.78) (end 110.4025 110.0606) (width 0.25) (layer "B.Cu") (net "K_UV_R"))
 (segment (start 113.3356 112.9217) (end 114 112.2573) (width 0.25) (layer "B.Cu") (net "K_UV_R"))
 (segment (start 112.8522 113.0419) (end 113.1353 113.0419) (width 0.1874) (layer "B.Cu") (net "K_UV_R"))
 (segment (start 111.6831 106.4598) (end 111.6831 108.78) (width 0.25) (layer "B.Cu") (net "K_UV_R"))
 (segment (start 110.4025 112.6726) (end 110.7718 113.0419) (width 0.25) (layer "B.Cu") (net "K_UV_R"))
 (segment (start 114 112.2573) (end 114 111.8) (width 0.25) (layer "B.Cu") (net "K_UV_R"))
 (segment (start 117.1256 105.5935) (end 118.0634 104.6557) (width 0.25) (layer "B.Cu") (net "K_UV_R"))
 (segment (start 111.6831 106.4598) (end 112.5494 105.5935) (width 0.25) (layer "B.Cu") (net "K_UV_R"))
 (segment (start 118.0634 104.6557) (end 118.0634 104.4391) (width 0.25) (layer "B.Cu") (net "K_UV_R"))
 (segment (start 112.5 105.5) (end 112.5 106.2767) (width 0.25) (layer "F.Cu") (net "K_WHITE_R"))
 (segment (start 112.5 106.2767) (end 115.3875 106.2767) (width 0.25) (layer "F.Cu") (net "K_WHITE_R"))
 (segment (start 115.3875 106.2767) (end 115.5 106.2767) (width 0.25) (layer "F.Cu") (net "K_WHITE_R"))
 (segment (start 115.5 105.5) (end 115.5 106.2767) (width 0.25) (layer "F.Cu") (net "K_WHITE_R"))
 (segment (start 115.3875 106.2767) (end 115.3875 106.4645) (width 0.25) (layer "F.Cu") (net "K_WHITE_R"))
 (via (at 115.3875 106.4645) (size 0.6) (drill 0.3) (layers "F.Cu" "B.Cu") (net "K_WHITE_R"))
 (segment (start 113 111.8) (end 113 108.852) (width 0.25) (layer "B.Cu") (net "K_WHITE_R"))
 (segment (start 113 108.852) (end 115.3875 106.4645) (width 0.25) (layer "B.Cu") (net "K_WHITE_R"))
 (segment (start 116 104.925) (end 116 106.4165) (width 0.25) (layer "F.Cu") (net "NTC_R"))
 (segment (start 116.0948 104.7233) (end 114.5 104.7233) (width 0.25) (layer "F.Cu") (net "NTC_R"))
 (segment (start 113.5 105.5) (end 114.5 105.5) (width 0.25) (layer "F.Cu") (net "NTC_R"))
 (segment (start 116.0999 104.7284) (end 116.0948 104.7233) (width 0.25) (layer "F.Cu") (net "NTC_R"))
 (segment (start 116 106.4165) (end 116.1525 106.569) (width 0.25) (layer "F.Cu") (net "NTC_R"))
 (segment (start 114.5 105.5) (end 114.5 104.7233) (width 0.25) (layer "F.Cu") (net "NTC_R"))
 (segment (start 116.0999 104.8251) (end 116.0999 104.7284) (width 0.1874) (layer "F.Cu") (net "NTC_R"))
 (segment (start 116 104.925) (end 116.0999 104.8251) (width 0.1874) (layer "F.Cu") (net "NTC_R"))
 (via (at 116.1525 106.569) (size 0.6) (drill 0.3) (layers "F.Cu" "B.Cu") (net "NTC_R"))
 (segment (start 115 107.7215) (end 116.1525 106.569) (width 0.25) (layer "B.Cu") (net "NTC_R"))
 (segment (start 115 111.8) (end 115 107.7215) (width 0.25) (layer "B.Cu") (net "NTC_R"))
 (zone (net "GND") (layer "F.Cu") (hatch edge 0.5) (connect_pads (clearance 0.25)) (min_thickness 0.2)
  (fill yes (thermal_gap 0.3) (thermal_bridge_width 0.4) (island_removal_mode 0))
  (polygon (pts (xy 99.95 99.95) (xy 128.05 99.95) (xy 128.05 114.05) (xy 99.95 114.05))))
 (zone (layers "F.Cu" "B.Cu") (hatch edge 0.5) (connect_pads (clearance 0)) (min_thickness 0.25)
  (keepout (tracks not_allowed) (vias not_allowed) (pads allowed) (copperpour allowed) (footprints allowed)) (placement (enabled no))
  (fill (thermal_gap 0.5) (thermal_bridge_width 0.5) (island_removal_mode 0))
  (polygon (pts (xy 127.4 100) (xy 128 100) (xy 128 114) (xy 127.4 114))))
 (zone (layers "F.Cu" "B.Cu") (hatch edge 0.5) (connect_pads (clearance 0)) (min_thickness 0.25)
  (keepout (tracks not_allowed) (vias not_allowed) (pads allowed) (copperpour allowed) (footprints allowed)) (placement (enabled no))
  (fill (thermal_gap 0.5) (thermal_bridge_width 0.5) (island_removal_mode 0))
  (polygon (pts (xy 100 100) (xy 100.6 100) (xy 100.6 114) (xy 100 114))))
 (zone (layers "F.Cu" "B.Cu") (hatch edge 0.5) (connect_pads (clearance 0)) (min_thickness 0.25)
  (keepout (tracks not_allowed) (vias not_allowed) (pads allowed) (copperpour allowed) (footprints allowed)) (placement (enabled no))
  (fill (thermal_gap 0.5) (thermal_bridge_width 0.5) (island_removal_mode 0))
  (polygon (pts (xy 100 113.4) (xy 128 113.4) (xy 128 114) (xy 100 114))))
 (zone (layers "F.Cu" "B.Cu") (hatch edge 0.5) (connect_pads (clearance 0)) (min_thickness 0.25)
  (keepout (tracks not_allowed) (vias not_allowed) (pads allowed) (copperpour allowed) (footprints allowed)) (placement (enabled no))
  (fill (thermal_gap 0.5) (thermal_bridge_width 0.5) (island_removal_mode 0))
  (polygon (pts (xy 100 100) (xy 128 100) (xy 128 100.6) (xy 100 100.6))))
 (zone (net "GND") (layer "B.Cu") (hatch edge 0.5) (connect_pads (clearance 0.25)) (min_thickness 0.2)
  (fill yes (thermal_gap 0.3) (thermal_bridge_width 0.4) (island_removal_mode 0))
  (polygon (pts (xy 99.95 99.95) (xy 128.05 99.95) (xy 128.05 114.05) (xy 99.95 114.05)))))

